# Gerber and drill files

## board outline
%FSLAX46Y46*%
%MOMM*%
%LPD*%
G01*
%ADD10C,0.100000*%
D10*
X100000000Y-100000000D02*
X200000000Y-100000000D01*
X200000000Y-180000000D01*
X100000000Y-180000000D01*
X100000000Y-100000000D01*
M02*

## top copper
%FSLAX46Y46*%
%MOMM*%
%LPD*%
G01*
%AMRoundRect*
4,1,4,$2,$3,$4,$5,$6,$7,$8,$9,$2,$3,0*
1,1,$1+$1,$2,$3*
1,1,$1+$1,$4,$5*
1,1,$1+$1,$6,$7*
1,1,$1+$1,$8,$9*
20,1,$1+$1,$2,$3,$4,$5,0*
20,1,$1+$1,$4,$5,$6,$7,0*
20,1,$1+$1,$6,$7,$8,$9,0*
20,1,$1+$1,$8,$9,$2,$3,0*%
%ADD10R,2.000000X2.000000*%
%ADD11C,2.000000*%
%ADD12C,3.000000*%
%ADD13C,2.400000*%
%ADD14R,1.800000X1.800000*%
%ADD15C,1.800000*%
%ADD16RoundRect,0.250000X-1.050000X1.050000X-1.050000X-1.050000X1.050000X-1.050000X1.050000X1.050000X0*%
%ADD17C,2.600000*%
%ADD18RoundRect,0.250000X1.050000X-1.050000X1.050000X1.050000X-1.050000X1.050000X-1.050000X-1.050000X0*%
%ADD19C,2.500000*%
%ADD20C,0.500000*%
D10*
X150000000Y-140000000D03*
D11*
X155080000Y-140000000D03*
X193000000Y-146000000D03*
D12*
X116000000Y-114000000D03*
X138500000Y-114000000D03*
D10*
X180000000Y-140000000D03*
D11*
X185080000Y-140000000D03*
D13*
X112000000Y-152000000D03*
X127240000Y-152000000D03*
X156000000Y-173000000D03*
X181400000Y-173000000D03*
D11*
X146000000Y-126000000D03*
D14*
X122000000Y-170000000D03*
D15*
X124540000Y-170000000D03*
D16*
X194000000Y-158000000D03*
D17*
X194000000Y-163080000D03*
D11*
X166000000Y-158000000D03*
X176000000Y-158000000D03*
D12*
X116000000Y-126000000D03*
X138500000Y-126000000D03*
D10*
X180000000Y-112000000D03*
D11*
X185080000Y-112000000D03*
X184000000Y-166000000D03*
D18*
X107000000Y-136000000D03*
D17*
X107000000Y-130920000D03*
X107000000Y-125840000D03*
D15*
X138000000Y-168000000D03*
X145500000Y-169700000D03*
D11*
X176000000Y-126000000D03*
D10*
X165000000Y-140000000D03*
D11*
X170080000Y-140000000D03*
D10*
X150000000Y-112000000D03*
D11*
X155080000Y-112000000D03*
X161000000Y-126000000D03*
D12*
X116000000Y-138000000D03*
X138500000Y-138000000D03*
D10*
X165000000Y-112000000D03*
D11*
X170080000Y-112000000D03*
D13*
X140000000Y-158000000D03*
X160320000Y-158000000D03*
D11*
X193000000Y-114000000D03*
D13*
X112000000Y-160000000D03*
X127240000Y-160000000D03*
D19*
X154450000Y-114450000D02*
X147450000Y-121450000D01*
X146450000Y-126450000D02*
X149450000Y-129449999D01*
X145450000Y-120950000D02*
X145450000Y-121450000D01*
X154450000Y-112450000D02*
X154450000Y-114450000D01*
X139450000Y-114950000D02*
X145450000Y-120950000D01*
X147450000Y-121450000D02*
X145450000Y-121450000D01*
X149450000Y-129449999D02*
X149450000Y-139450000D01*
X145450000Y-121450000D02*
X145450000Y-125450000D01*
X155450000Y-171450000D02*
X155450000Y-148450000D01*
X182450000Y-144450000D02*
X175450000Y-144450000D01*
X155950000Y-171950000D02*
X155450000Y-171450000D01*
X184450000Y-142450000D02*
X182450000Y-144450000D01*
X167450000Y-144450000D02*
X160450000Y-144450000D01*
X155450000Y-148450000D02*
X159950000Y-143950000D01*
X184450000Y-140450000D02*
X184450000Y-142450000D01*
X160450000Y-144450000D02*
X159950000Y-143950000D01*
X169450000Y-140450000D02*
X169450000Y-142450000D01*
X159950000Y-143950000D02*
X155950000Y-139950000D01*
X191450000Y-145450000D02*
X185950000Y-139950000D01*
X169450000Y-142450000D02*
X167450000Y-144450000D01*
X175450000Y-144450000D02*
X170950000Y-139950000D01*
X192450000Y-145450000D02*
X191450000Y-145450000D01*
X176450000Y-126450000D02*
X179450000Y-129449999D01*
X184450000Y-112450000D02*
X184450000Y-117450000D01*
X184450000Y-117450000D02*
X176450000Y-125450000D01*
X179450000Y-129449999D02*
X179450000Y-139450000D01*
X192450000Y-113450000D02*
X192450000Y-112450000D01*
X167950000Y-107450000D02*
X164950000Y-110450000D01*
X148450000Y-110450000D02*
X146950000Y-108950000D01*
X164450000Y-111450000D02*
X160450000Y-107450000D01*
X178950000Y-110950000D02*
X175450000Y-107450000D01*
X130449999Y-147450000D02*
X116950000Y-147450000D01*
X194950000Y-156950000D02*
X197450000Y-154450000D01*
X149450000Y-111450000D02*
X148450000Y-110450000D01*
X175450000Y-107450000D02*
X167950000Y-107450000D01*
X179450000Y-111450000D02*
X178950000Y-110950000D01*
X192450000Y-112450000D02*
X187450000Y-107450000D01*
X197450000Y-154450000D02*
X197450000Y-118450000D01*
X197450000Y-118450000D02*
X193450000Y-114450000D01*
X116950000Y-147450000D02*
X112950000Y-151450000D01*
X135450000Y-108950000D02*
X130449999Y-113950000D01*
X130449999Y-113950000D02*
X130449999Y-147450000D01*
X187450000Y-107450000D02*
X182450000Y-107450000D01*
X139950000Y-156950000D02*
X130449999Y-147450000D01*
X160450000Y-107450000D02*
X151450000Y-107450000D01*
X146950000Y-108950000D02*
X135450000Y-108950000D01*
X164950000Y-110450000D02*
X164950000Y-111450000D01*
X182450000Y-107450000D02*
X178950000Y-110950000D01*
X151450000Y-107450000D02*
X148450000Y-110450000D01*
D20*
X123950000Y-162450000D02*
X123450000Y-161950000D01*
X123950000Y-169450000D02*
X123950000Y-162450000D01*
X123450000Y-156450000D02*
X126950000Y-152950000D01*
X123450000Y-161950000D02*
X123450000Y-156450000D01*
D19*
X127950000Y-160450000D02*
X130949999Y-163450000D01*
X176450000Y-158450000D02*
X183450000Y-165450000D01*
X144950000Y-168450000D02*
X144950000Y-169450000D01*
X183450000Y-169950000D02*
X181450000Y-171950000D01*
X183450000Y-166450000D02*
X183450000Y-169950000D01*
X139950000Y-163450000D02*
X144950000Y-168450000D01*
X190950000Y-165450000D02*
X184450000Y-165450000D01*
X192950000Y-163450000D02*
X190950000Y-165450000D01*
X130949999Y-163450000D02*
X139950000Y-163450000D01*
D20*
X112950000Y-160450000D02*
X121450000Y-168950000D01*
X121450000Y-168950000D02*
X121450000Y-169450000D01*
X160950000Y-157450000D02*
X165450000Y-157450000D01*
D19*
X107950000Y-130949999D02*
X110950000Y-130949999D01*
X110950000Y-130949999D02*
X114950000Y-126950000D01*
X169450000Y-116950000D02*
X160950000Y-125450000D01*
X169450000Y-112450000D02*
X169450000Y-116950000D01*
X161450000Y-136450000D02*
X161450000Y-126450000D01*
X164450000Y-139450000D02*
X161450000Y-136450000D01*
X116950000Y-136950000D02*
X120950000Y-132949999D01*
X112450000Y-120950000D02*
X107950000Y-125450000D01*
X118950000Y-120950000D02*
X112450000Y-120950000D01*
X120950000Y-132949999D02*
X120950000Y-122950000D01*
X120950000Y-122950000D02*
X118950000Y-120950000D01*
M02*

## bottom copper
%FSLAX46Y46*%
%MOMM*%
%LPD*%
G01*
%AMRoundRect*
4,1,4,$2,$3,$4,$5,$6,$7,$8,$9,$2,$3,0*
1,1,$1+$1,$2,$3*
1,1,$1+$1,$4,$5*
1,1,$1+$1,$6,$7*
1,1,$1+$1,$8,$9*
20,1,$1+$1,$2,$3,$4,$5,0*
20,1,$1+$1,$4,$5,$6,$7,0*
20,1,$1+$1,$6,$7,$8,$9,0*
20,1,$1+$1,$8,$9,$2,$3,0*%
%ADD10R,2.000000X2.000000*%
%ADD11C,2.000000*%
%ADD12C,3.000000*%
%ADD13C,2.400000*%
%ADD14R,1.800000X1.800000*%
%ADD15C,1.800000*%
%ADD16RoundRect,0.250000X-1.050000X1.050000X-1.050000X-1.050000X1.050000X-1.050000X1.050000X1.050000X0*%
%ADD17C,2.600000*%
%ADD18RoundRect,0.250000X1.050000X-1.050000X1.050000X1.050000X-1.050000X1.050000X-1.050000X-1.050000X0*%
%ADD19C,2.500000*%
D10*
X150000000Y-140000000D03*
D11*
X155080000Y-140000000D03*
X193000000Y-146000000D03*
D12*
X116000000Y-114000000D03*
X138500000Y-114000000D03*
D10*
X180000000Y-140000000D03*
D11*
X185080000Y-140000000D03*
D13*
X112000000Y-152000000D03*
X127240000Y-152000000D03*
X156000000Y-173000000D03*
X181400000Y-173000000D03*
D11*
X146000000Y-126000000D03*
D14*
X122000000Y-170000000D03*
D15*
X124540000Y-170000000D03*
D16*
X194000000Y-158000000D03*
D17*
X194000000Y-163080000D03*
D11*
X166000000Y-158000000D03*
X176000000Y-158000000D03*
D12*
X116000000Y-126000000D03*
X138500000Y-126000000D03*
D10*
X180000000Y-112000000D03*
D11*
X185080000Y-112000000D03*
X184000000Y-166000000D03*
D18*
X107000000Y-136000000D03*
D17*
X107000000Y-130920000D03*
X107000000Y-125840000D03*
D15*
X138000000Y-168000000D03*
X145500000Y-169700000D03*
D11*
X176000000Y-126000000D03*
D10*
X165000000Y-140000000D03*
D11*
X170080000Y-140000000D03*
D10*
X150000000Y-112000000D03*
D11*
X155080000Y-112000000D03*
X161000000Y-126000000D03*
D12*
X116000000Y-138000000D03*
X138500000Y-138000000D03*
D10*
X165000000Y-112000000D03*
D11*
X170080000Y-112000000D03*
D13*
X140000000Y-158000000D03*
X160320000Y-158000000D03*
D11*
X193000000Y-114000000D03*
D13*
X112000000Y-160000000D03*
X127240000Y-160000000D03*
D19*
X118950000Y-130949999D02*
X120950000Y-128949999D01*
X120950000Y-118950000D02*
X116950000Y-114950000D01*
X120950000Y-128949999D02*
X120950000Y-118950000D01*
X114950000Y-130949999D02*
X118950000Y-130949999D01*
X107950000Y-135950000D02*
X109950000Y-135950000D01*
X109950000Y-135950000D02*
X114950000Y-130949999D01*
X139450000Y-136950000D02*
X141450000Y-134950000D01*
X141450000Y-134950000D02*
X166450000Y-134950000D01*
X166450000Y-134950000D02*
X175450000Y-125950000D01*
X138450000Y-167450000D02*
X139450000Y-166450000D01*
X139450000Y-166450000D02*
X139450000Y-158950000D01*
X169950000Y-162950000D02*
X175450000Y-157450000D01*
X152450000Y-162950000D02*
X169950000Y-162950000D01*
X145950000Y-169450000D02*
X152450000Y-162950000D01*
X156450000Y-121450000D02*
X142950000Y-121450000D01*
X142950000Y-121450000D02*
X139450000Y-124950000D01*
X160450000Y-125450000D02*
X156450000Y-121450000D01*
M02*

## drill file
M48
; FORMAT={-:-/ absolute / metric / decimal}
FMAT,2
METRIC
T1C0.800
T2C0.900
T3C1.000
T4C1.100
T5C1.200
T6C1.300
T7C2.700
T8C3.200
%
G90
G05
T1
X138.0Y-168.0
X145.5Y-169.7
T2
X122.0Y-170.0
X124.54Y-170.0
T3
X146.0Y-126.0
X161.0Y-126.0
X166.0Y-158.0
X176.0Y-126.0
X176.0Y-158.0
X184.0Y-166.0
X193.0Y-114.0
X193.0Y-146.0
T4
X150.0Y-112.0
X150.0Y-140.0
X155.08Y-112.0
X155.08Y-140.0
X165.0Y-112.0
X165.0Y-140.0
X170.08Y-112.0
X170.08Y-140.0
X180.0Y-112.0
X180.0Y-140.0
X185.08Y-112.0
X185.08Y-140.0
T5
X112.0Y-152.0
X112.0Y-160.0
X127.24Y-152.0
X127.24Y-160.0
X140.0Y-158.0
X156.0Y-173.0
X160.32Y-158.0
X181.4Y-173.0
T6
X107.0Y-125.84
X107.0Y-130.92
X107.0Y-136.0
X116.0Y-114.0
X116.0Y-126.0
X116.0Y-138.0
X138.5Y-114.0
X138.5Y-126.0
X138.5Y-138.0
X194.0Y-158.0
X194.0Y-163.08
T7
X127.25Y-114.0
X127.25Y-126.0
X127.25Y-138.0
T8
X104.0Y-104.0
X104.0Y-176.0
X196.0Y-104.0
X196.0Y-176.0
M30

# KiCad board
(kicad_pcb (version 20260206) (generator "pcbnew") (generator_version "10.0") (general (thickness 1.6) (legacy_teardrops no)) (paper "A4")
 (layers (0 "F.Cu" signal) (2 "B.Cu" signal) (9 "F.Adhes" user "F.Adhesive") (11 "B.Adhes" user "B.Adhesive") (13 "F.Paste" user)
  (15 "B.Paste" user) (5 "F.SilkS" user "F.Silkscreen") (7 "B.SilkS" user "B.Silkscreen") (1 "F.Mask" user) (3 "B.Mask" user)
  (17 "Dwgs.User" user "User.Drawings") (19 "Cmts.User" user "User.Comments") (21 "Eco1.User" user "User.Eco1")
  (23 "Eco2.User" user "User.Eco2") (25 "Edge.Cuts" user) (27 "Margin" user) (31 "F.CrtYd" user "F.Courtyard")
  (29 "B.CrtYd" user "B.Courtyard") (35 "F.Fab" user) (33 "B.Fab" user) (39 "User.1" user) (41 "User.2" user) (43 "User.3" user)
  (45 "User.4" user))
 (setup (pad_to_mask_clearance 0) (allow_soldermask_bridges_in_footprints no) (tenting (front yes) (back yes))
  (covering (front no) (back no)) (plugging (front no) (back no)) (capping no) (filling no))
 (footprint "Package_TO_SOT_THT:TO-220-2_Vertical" (layer "F.Cu") (at 150 140)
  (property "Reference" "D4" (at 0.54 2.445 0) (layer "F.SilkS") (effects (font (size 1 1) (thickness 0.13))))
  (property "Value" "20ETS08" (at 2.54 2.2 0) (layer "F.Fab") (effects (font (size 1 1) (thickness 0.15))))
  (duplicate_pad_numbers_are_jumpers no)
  (pad "1" thru_hole rect (at 0 0) (size 2 2) (drill 1.1) (layers "*.Cu" "*.Mask") (remove_unused_layers no) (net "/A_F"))
  (pad "2" thru_hole circle (at 5.08 0) (size 2 2) (drill 1.1) (layers "*.Cu" "*.Mask") (remove_unused_layers no) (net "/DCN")))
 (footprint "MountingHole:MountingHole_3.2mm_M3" (layer "F.Cu") (at 104 176)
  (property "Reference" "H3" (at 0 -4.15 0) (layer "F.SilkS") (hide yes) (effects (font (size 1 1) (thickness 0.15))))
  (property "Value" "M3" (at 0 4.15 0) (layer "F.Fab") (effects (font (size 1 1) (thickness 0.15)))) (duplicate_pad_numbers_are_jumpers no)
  (pad "" np_thru_hole circle (at 0 0) (size 3.2 3.2) (drill 3.2) (layers "*.Cu" "*.Mask")))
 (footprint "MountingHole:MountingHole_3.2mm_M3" (layer "F.Cu") (at 104 104)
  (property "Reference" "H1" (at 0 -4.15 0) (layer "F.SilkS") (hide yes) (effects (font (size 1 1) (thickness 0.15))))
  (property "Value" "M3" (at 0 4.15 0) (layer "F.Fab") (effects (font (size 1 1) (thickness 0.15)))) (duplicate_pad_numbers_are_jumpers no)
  (pad "" np_thru_hole circle (at 0 0) (size 3.2 3.2) (drill 3.2) (layers "*.Cu" "*.Mask")))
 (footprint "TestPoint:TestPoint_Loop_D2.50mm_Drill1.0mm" (layer "F.Cu") (at 193 146)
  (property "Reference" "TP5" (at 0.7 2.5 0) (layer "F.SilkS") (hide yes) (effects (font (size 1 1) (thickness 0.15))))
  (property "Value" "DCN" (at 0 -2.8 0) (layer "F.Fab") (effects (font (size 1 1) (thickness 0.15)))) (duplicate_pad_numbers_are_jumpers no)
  (pad "1" thru_hole circle (at 0 0) (size 2 2) (drill 1) (layers "*.Cu" "*.Mask") (remove_unused_layers no) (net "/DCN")))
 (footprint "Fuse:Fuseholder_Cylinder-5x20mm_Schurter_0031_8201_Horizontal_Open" (layer "F.Cu") (at 116 114)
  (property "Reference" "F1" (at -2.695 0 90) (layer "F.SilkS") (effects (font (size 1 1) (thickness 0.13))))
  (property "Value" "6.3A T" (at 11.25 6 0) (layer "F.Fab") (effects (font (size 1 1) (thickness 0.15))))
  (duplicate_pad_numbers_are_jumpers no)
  (pad "" np_thru_hole circle (at 11.25 0) (size 2.7 2.7) (drill 2.7) (layers "*.Cu" "*.Mask"))
  (pad "1" thru_hole circle (at 0 0) (size 3 3) (drill 1.3) (layers "*.Cu" "*.Mask") (remove_unused_layers no) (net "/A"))
  (pad "2" thru_hole circle (at 22.5 0) (size 3 3) (drill 1.3) (layers "*.Cu" "*.Mask") (remove_unused_layers no) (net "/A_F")))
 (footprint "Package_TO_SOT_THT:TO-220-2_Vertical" (layer "F.Cu") (at 180 140)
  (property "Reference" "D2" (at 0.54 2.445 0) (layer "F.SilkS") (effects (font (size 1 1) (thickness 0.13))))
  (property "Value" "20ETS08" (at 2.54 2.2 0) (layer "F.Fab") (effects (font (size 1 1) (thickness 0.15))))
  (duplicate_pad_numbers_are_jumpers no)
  (pad "1" thru_hole rect (at 0 0) (size 2 2) (drill 1.1) (layers "*.Cu" "*.Mask") (remove_unused_layers no) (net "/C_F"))
  (pad "2" thru_hole circle (at 5.08 0) (size 2 2) (drill 1.1) (layers "*.Cu" "*.Mask") (remove_unused_layers no) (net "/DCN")))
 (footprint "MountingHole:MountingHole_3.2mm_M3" (layer "F.Cu") (at 196 176)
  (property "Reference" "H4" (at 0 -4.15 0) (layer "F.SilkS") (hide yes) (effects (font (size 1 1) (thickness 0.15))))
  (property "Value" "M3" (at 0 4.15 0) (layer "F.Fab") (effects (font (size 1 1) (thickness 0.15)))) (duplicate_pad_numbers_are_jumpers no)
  (pad "" np_thru_hole circle (at 0 0) (size 3.2 3.2) (drill 3.2) (layers "*.Cu" "*.Mask")))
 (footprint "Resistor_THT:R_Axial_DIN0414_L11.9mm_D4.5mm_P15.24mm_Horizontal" (layer "F.Cu") (at 112 152)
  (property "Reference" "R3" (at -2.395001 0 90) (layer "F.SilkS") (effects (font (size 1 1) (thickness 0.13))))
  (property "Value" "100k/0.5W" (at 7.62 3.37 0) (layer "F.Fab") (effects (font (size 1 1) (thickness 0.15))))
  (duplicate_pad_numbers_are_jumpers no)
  (pad "1" thru_hole circle (at 0 0) (size 2.4 2.4) (drill 1.2) (layers "*.Cu" "*.Mask") (remove_unused_layers no) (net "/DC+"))
  (pad "2" thru_hole circle (at 15.24 0) (size 2.4 2.4) (drill 1.2) (layers "*.Cu" "*.Mask") (remove_unused_layers no) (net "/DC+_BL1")))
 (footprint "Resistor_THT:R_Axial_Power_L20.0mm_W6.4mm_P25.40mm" (layer "F.Cu") (at 156 173)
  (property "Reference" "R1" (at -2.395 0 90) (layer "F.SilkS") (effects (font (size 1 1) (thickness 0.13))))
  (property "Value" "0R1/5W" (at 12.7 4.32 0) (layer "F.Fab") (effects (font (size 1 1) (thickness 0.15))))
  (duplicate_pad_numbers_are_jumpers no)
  (pad "1" thru_hole circle (at 0 0) (size 2.4 2.4) (drill 1.2) (layers "*.Cu" "*.Mask") (remove_unused_layers no) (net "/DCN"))
  (pad "2" thru_hole circle (at 25.4 0) (size 2.4 2.4) (drill 1.2) (layers "*.Cu" "*.Mask") (remove_unused_layers no) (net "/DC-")))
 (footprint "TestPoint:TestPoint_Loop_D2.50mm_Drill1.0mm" (layer "F.Cu") (at 146 126)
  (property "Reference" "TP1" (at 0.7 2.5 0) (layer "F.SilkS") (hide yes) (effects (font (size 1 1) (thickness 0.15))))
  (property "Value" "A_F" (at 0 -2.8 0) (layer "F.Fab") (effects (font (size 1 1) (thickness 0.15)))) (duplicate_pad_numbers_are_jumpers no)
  (pad "1" thru_hole circle (at 0 0) (size 2 2) (drill 1) (layers "*.Cu" "*.Mask") (remove_unused_layers no) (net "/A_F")))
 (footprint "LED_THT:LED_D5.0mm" (layer "F.Cu") (at 122 170)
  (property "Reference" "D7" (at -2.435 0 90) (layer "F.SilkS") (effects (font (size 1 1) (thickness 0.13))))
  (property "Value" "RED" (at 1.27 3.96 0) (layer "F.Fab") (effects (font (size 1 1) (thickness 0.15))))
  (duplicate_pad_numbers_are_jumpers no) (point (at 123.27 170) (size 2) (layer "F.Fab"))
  (pad "1" thru_hole rect (at 0 0) (size 1.8 1.8) (drill 0.9) (layers "*.Cu" "*.Mask") (remove_unused_layers no) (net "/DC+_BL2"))
  (pad "2" thru_hole circle (at 2.54 0) (size 1.8 1.8) (drill 0.9) (layers "*.Cu" "*.Mask") (remove_unused_layers no) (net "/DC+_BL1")))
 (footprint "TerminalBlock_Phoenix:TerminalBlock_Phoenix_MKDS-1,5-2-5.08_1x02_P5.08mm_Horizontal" (layer "F.Cu") (at 194 158 -90)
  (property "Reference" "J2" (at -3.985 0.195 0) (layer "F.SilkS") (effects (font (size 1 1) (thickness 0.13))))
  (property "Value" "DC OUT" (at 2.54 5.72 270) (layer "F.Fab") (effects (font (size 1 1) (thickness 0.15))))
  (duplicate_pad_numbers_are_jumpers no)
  (pad "1" thru_hole roundrect (at 0 0 270) (size 2.6 2.6) (drill 1.3) (layers "*.Cu" "*.Mask") (remove_unused_layers no)
   (roundrect_rratio 0.096154) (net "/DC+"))
  (pad "2" thru_hole circle (at 5.08 0 270) (size 2.6 2.6) (drill 1.3) (layers "*.Cu" "*.Mask") (remove_unused_layers no) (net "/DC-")))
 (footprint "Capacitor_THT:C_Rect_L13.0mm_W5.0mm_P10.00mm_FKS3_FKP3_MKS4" (layer "F.Cu") (at 166 158)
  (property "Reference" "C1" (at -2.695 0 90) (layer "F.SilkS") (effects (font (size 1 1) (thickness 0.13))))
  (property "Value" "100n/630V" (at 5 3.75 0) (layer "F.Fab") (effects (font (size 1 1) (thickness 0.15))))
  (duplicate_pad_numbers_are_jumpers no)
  (pad "1" thru_hole circle (at 0 0) (size 2 2) (drill 1) (layers "*.Cu" "*.Mask") (remove_unused_layers no) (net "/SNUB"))
  (pad "2" thru_hole circle (at 10 0) (size 2 2) (drill 1) (layers "*.Cu" "*.Mask") (remove_unused_layers no) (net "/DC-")))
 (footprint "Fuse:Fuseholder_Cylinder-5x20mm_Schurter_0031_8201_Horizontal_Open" (layer "F.Cu") (at 116 126)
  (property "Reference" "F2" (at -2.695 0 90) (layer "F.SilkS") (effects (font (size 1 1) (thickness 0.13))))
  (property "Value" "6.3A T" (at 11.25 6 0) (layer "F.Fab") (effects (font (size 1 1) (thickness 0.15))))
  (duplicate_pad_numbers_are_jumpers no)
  (pad "" np_thru_hole circle (at 11.25 0) (size 2.7 2.7) (drill 2.7) (layers "*.Cu" "*.Mask"))
  (pad "1" thru_hole circle (at 0 0) (size 3 3) (drill 1.3) (layers "*.Cu" "*.Mask") (remove_unused_layers no) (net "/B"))
  (pad "2" thru_hole circle (at 22.5 0) (size 3 3) (drill 1.3) (layers "*.Cu" "*.Mask") (remove_unused_layers no) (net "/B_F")))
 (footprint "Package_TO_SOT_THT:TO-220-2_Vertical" (layer "F.Cu") (at 180 112)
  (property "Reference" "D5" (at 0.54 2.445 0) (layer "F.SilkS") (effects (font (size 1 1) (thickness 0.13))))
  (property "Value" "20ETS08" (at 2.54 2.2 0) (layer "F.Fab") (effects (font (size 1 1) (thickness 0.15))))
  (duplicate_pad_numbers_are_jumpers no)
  (pad "1" thru_hole rect (at 0 0) (size 2 2) (drill 1.1) (layers "*.Cu" "*.Mask") (remove_unused_layers no) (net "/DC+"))
  (pad "2" thru_hole circle (at 5.08 0) (size 2 2) (drill 1.1) (layers "*.Cu" "*.Mask") (remove_unused_layers no) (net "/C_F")))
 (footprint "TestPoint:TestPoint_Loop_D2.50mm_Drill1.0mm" (layer "F.Cu") (at 184 166)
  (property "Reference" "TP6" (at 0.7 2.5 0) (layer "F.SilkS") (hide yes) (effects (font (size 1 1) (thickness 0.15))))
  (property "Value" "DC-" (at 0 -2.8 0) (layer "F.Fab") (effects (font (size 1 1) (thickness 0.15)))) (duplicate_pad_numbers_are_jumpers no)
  (pad "1" thru_hole circle (at 0 0) (size 2 2) (drill 1) (layers "*.Cu" "*.Mask") (remove_unused_layers no) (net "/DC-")))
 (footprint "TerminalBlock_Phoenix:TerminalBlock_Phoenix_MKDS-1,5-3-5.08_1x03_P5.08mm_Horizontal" (layer "F.Cu") (at 107 136 90)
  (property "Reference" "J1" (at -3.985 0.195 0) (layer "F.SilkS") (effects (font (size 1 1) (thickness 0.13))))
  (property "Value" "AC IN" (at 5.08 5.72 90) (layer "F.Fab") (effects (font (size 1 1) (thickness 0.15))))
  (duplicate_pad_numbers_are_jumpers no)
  (pad "1" thru_hole roundrect (at 0 0 90) (size 2.6 2.6) (drill 1.3) (layers "*.Cu" "*.Mask") (remove_unused_layers no)
   (roundrect_rratio 0.096154) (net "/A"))
  (pad "2" thru_hole circle (at 5.08 0 90) (size 2.6 2.6) (drill 1.3) (layers "*.Cu" "*.Mask") (remove_unused_layers no) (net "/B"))
  (pad "3" thru_hole circle (at 10.16 0 90) (size 2.6 2.6) (drill 1.3) (layers "*.Cu" "*.Mask") (remove_unused_layers no) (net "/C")))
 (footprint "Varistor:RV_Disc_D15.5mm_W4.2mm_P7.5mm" (layer "F.Cu") (at 138 168)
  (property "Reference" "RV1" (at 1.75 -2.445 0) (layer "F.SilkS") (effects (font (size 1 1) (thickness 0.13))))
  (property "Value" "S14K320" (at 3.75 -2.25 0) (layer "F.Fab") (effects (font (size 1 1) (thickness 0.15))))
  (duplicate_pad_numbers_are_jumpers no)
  (pad "1" thru_hole circle (at 0 0) (size 1.8 1.8) (drill 0.8) (layers "*.Cu" "*.Mask") (remove_unused_layers no) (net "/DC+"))
  (pad "2" thru_hole circle (at 7.5 1.7) (size 1.8 1.8) (drill 0.8) (layers "*.Cu" "*.Mask") (remove_unused_layers no) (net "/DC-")))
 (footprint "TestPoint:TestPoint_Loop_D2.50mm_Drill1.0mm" (layer "F.Cu") (at 176 126)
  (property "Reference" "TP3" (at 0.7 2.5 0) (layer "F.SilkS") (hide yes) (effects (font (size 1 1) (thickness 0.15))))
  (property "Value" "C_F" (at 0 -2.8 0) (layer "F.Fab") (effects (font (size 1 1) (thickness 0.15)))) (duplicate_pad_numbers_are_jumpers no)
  (pad "1" thru_hole circle (at 0 0) (size 2 2) (drill 1) (layers "*.Cu" "*.Mask") (remove_unused_layers no) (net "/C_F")))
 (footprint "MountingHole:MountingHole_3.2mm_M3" (layer "F.Cu") (at 196 104)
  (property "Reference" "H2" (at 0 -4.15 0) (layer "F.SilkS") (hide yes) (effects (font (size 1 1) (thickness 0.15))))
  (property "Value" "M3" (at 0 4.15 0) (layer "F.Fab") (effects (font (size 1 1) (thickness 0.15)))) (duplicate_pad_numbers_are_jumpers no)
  (pad "" np_thru_hole circle (at 0 0) (size 3.2 3.2) (drill 3.2) (layers "*.Cu" "*.Mask")))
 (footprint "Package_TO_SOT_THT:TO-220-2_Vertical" (layer "F.Cu") (at 165 140)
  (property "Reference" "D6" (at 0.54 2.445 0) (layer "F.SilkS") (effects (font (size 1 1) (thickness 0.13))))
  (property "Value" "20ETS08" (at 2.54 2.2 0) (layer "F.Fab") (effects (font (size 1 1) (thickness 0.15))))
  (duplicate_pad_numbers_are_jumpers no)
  (pad "1" thru_hole rect (at 0 0) (size 2 2) (drill 1.1) (layers "*.Cu" "*.Mask") (remove_unused_layers no) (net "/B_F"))
  (pad "2" thru_hole circle (at 5.08 0) (size 2 2) (drill 1.1) (layers "*.Cu" "*.Mask") (remove_unused_layers no) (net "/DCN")))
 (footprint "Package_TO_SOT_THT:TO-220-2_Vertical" (layer "F.Cu") (at 150 112)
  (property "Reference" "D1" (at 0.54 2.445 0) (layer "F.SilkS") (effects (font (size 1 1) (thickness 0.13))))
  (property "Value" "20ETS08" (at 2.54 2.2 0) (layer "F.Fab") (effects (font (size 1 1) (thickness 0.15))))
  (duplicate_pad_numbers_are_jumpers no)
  (pad "1" thru_hole rect (at 0 0) (size 2 2) (drill 1.1) (layers "*.Cu" "*.Mask") (remove_unused_layers no) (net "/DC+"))
  (pad "2" thru_hole circle (at 5.08 0) (size 2 2) (drill 1.1) (layers "*.Cu" "*.Mask") (remove_unused_layers no) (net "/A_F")))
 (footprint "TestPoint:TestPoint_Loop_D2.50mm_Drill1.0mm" (layer "F.Cu") (at 161 126)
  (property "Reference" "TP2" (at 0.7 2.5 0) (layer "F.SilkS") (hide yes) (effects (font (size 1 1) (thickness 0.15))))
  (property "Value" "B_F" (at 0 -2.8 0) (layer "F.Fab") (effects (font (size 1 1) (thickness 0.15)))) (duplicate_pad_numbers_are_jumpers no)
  (pad "1" thru_hole circle (at 0 0) (size 2 2) (drill 1) (layers "*.Cu" "*.Mask") (remove_unused_layers no) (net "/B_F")))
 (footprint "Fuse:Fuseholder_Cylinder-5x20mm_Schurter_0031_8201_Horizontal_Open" (layer "F.Cu") (at 116 138)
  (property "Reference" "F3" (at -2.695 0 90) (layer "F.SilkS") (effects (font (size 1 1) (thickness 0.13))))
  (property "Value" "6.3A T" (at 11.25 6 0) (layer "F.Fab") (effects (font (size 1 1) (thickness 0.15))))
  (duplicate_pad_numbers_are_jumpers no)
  (pad "" np_thru_hole circle (at 11.25 0) (size 2.7 2.7) (drill 2.7) (layers "*.Cu" "*.Mask"))
  (pad "1" thru_hole circle (at 0 0) (size 3 3) (drill 1.3) (layers "*.Cu" "*.Mask") (remove_unused_layers no) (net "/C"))
  (pad "2" thru_hole circle (at 22.5 0) (size 3 3) (drill 1.3) (layers "*.Cu" "*.Mask") (remove_unused_layers no) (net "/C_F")))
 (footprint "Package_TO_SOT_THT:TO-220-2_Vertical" (layer "F.Cu") (at 165 112)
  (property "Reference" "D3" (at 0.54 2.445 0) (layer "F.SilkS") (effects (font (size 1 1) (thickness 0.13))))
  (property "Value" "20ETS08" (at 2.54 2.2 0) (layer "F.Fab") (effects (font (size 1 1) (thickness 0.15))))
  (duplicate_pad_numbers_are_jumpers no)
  (pad "1" thru_hole rect (at 0 0) (size 2 2) (drill 1.1) (layers "*.Cu" "*.Mask") (remove_unused_layers no) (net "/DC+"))
  (pad "2" thru_hole circle (at 5.08 0) (size 2 2) (drill 1.1) (layers "*.Cu" "*.Mask") (remove_unused_layers no) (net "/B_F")))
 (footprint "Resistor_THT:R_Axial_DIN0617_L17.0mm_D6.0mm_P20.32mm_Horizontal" (layer "F.Cu") (at 140 158)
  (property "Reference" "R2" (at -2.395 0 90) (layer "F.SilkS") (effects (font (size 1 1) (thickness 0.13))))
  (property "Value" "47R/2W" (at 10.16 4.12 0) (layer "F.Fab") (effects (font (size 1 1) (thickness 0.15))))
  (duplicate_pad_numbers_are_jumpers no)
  (pad "1" thru_hole circle (at 0 0) (size 2.4 2.4) (drill 1.2) (layers "*.Cu" "*.Mask") (remove_unused_layers no) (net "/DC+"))
  (pad "2" thru_hole circle (at 20.32 0) (size 2.4 2.4) (drill 1.2) (layers "*.Cu" "*.Mask") (remove_unused_layers no) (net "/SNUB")))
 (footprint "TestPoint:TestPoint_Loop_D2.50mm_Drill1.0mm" (layer "F.Cu") (at 193 114)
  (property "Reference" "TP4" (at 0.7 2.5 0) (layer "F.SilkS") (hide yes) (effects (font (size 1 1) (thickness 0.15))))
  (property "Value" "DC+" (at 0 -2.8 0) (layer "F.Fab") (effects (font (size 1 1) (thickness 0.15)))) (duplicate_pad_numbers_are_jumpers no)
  (pad "1" thru_hole circle (at 0 0) (size 2 2) (drill 1) (layers "*.Cu" "*.Mask") (remove_unused_layers no) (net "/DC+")))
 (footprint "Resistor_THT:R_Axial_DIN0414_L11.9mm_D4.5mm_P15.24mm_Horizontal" (layer "F.Cu") (at 112 160)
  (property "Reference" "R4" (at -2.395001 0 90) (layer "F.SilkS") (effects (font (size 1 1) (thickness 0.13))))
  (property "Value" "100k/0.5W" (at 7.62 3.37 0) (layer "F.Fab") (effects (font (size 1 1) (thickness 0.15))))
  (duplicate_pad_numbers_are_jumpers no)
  (pad "1" thru_hole circle (at 0 0) (size 2.4 2.4) (drill 1.2) (layers "*.Cu" "*.Mask") (remove_unused_layers no) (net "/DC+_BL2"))
  (pad "2" thru_hole circle (at 15.24 0) (size 2.4 2.4) (drill 1.2) (layers "*.Cu" "*.Mask") (remove_unused_layers no) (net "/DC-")))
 (gr_rect (start 100 100) (end 200 180) (stroke (width 0.1) (type default)) (fill no) (layer "Edge.Cuts"))
 (segment (start 154.45 114.45) (end 147.45 121.45) (width 2.5) (layer "F.Cu") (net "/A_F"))
 (segment (start 146.45 126.45) (end 149.45 129.449999) (width 2.5) (layer "F.Cu") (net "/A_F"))
 (segment (start 145.45 120.95) (end 145.45 121.45) (width 2.5) (layer "F.Cu") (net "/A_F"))
 (segment (start 154.45 112.45) (end 154.45 114.45) (width 2.5) (layer "F.Cu") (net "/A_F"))
 (segment (start 139.45 114.95) (end 145.45 120.95) (width 2.5) (layer "F.Cu") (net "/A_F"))
 (segment (start 147.45 121.45) (end 145.45 121.45) (width 2.5) (layer "F.Cu") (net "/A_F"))
 (segment (start 149.45 129.449999) (end 149.45 139.45) (width 2.5) (layer "F.Cu") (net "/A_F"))
 (segment (start 145.45 121.45) (end 145.45 125.45) (width 2.5) (layer "F.Cu") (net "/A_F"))
 (segment (start 155.45 171.45) (end 155.45 148.45) (width 2.5) (layer "F.Cu") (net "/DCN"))
 (segment (start 182.45 144.45) (end 175.45 144.45) (width 2.5) (layer "F.Cu") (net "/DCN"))
 (segment (start 155.95 171.95) (end 155.45 171.45) (width 2.5) (layer "F.Cu") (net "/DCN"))
 (segment (start 184.45 142.45) (end 182.45 144.45) (width 2.5) (layer "F.Cu") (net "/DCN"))
 (segment (start 167.45 144.45) (end 160.45 144.45) (width 2.5) (layer "F.Cu") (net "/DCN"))
 (segment (start 155.45 148.45) (end 159.95 143.95) (width 2.5) (layer "F.Cu") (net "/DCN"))
 (segment (start 184.45 140.45) (end 184.45 142.45) (width 2.5) (layer "F.Cu") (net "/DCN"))
 (segment (start 160.45 144.45) (end 159.95 143.95) (width 2.5) (layer "F.Cu") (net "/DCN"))
 (segment (start 169.45 140.45) (end 169.45 142.45) (width 2.5) (layer "F.Cu") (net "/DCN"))
 (segment (start 159.95 143.95) (end 155.95 139.95) (width 2.5) (layer "F.Cu") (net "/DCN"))
 (segment (start 191.45 145.45) (end 185.95 139.95) (width 2.5) (layer "F.Cu") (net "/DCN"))
 (segment (start 169.45 142.45) (end 167.45 144.45) (width 2.5) (layer "F.Cu") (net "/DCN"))
 (segment (start 175.45 144.45) (end 170.95 139.95) (width 2.5) (layer "F.Cu") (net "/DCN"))
 (segment (start 192.45 145.45) (end 191.45 145.45) (width 2.5) (layer "F.Cu") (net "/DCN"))
 (segment (start 118.95 130.949999) (end 120.95 128.949999) (width 2.5) (layer "B.Cu") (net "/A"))
 (segment (start 120.95 118.95) (end 116.95 114.95) (width 2.5) (layer "B.Cu") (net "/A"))
 (segment (start 120.95 128.949999) (end 120.95 118.95) (width 2.5) (layer "B.Cu") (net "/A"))
 (segment (start 114.95 130.949999) (end 118.95 130.949999) (width 2.5) (layer "B.Cu") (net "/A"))
 (segment (start 107.95 135.95) (end 109.95 135.95) (width 2.5) (layer "B.Cu") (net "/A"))
 (segment (start 109.95 135.95) (end 114.95 130.949999) (width 2.5) (layer "B.Cu") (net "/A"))
 (segment (start 176.45 126.45) (end 179.45 129.449999) (width 2.5) (layer "F.Cu") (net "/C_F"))
 (segment (start 184.45 112.45) (end 184.45 117.45) (width 2.5) (layer "F.Cu") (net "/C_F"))
 (segment (start 184.45 117.45) (end 176.45 125.45) (width 2.5) (layer "F.Cu") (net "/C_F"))
 (segment (start 179.45 129.449999) (end 179.45 139.45) (width 2.5) (layer "F.Cu") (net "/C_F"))
 (segment (start 139.45 136.95) (end 141.45 134.95) (width 2.5) (layer "B.Cu") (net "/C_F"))
 (segment (start 141.45 134.95) (end 166.45 134.95) (width 2.5) (layer "B.Cu") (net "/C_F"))
 (segment (start 166.45 134.95) (end 175.45 125.95) (width 2.5) (layer "B.Cu") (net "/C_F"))
 (segment (start 192.45 113.45) (end 192.45 112.45) (width 2.5) (layer "F.Cu") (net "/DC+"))
 (segment (start 167.95 107.45) (end 164.95 110.45) (width 2.5) (layer "F.Cu") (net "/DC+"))
 (segment (start 148.45 110.45) (end 146.95 108.95) (width 2.5) (layer "F.Cu") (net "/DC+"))
 (segment (start 164.45 111.45) (end 160.45 107.45) (width 2.5) (layer "F.Cu") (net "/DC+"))
 (segment (start 178.95 110.95) (end 175.45 107.45) (width 2.5) (layer "F.Cu") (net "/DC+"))
 (segment (start 130.449999 147.45) (end 116.95 147.45) (width 2.5) (layer "F.Cu") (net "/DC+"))
 (segment (start 194.95 156.95) (end 197.45 154.45) (width 2.5) (layer "F.Cu") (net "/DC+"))
 (segment (start 149.45 111.45) (end 148.45 110.45) (width 2.5) (layer "F.Cu") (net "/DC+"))
 (segment (start 175.45 107.45) (end 167.95 107.45) (width 2.5) (layer "F.Cu") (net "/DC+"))
 (segment (start 179.45 111.45) (end 178.95 110.95) (width 2.5) (layer "F.Cu") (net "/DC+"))
 (segment (start 192.45 112.45) (end 187.45 107.45) (width 2.5) (layer "F.Cu") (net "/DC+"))
 (segment (start 197.45 154.45) (end 197.45 118.45) (width 2.5) (layer "F.Cu") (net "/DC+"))
 (segment (start 197.45 118.45) (end 193.45 114.45) (width 2.5) (layer "F.Cu") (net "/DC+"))
 (segment (start 116.95 147.45) (end 112.95 151.45) (width 2.5) (layer "F.Cu") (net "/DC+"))
 (segment (start 135.45 108.95) (end 130.449999 113.95) (width 2.5) (layer "F.Cu") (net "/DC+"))
 (segment (start 130.449999 113.95) (end 130.449999 147.45) (width 2.5) (layer "F.Cu") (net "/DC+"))
 (segment (start 187.45 107.45) (end 182.45 107.45) (width 2.5) (layer "F.Cu") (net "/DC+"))
 (segment (start 139.95 156.95) (end 130.449999 147.45) (width 2.5) (layer "F.Cu") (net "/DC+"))
 (segment (start 160.45 107.45) (end 151.45 107.45) (width 2.5) (layer "F.Cu") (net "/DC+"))
 (segment (start 146.95 108.95) (end 135.45 108.95) (width 2.5) (layer "F.Cu") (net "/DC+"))
 (segment (start 164.95 110.45) (end 164.95 111.45) (width 2.5) (layer "F.Cu") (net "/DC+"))
 (segment (start 182.45 107.45) (end 178.95 110.95) (width 2.5) (layer "F.Cu") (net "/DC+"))
 (segment (start 151.45 107.45) (end 148.45 110.45) (width 2.5) (layer "F.Cu") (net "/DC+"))
 (segment (start 138.45 167.45) (end 139.45 166.45) (width 2.5) (layer "B.Cu") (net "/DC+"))
 (segment (start 139.45 166.45) (end 139.45 158.95) (width 2.5) (layer "B.Cu") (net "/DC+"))
 (segment (start 123.95 162.45) (end 123.45 161.95) (width 0.5) (layer "F.Cu") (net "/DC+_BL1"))
 (segment (start 123.95 169.45) (end 123.95 162.45) (width 0.5) (layer "F.Cu") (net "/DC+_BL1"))
 (segment (start 123.45 156.45) (end 126.95 152.95) (width 0.5) (layer "F.Cu") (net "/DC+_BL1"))
 (segment (start 123.45 161.95) (end 123.45 156.45) (width 0.5) (layer "F.Cu") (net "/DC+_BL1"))
 (segment (start 127.95 160.45) (end 130.949999 163.45) (width 2.5) (layer "F.Cu") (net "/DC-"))
 (segment (start 176.45 158.45) (end 183.45 165.45) (width 2.5) (layer "F.Cu") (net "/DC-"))
 (segment (start 144.95 168.45) (end 144.95 169.45) (width 2.5) (layer "F.Cu") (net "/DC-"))
 (segment (start 183.45 169.95) (end 181.45 171.95) (width 2.5) (layer "F.Cu") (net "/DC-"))
 (segment (start 183.45 166.45) (end 183.45 169.95) (width 2.5) (layer "F.Cu") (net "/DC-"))
 (segment (start 139.95 163.45) (end 144.95 168.45) (width 2.5) (layer "F.Cu") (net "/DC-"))
 (segment (start 190.95 165.45) (end 184.45 165.45) (width 2.5) (layer "F.Cu") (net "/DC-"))
 (segment (start 192.95 163.45) (end 190.95 165.45) (width 2.5) (layer "F.Cu") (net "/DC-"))
 (segment (start 130.949999 163.45) (end 139.95 163.45) (width 2.5) (layer "F.Cu") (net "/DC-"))
 (segment (start 169.95 162.95) (end 175.45 157.45) (width 2.5) (layer "B.Cu") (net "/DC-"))
 (segment (start 152.45 162.95) (end 169.95 162.95) (width 2.5) (layer "B.Cu") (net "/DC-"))
 (segment (start 145.95 169.45) (end 152.45 162.95) (width 2.5) (layer "B.Cu") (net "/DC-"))
 (segment (start 112.95 160.45) (end 121.45 168.95) (width 0.5) (layer "F.Cu") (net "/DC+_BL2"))
 (segment (start 121.45 168.95) (end 121.45 169.45) (width 0.5) (layer "F.Cu") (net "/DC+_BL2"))
 (segment (start 160.95 157.45) (end 165.45 157.45) (width 0.5) (layer "F.Cu") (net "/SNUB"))
 (segment (start 107.95 130.949999) (end 110.95 130.949999) (width 2.5) (layer "F.Cu") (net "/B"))
 (segment (start 110.95 130.949999) (end 114.95 126.95) (width 2.5) (layer "F.Cu") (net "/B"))
 (segment (start 169.45 116.95) (end 160.95 125.45) (width 2.5) (layer "F.Cu") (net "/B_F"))
 (segment (start 169.45 112.45) (end 169.45 116.95) (width 2.5) (layer "F.Cu") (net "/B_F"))
 (segment (start 161.45 136.45) (end 161.45 126.45) (width 2.5) (layer "F.Cu") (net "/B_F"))
 (segment (start 164.45 139.45) (end 161.45 136.45) (width 2.5) (layer "F.Cu") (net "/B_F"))
 (segment (start 156.45 121.45) (end 142.95 121.45) (width 2.5) (layer "B.Cu") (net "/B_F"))
 (segment (start 142.95 121.45) (end 139.45 124.95) (width 2.5) (layer "B.Cu") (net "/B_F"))
 (segment (start 160.45 125.45) (end 156.45 121.45) (width 2.5) (layer "B.Cu") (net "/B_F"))
 (segment (start 116.95 136.95) (end 120.95 132.949999) (width 2.5) (layer "F.Cu") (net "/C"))
 (segment (start 112.45 120.95) (end 107.95 125.45) (width 2.5) (layer "F.Cu") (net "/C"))
 (segment (start 118.95 120.95) (end 112.45 120.95) (width 2.5) (layer "F.Cu") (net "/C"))
 (segment (start 120.95 132.949999) (end 120.95 122.95) (width 2.5) (layer "F.Cu") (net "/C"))
 (segment (start 120.95 122.95) (end 118.95 120.95) (width 2.5) (layer "F.Cu") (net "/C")))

